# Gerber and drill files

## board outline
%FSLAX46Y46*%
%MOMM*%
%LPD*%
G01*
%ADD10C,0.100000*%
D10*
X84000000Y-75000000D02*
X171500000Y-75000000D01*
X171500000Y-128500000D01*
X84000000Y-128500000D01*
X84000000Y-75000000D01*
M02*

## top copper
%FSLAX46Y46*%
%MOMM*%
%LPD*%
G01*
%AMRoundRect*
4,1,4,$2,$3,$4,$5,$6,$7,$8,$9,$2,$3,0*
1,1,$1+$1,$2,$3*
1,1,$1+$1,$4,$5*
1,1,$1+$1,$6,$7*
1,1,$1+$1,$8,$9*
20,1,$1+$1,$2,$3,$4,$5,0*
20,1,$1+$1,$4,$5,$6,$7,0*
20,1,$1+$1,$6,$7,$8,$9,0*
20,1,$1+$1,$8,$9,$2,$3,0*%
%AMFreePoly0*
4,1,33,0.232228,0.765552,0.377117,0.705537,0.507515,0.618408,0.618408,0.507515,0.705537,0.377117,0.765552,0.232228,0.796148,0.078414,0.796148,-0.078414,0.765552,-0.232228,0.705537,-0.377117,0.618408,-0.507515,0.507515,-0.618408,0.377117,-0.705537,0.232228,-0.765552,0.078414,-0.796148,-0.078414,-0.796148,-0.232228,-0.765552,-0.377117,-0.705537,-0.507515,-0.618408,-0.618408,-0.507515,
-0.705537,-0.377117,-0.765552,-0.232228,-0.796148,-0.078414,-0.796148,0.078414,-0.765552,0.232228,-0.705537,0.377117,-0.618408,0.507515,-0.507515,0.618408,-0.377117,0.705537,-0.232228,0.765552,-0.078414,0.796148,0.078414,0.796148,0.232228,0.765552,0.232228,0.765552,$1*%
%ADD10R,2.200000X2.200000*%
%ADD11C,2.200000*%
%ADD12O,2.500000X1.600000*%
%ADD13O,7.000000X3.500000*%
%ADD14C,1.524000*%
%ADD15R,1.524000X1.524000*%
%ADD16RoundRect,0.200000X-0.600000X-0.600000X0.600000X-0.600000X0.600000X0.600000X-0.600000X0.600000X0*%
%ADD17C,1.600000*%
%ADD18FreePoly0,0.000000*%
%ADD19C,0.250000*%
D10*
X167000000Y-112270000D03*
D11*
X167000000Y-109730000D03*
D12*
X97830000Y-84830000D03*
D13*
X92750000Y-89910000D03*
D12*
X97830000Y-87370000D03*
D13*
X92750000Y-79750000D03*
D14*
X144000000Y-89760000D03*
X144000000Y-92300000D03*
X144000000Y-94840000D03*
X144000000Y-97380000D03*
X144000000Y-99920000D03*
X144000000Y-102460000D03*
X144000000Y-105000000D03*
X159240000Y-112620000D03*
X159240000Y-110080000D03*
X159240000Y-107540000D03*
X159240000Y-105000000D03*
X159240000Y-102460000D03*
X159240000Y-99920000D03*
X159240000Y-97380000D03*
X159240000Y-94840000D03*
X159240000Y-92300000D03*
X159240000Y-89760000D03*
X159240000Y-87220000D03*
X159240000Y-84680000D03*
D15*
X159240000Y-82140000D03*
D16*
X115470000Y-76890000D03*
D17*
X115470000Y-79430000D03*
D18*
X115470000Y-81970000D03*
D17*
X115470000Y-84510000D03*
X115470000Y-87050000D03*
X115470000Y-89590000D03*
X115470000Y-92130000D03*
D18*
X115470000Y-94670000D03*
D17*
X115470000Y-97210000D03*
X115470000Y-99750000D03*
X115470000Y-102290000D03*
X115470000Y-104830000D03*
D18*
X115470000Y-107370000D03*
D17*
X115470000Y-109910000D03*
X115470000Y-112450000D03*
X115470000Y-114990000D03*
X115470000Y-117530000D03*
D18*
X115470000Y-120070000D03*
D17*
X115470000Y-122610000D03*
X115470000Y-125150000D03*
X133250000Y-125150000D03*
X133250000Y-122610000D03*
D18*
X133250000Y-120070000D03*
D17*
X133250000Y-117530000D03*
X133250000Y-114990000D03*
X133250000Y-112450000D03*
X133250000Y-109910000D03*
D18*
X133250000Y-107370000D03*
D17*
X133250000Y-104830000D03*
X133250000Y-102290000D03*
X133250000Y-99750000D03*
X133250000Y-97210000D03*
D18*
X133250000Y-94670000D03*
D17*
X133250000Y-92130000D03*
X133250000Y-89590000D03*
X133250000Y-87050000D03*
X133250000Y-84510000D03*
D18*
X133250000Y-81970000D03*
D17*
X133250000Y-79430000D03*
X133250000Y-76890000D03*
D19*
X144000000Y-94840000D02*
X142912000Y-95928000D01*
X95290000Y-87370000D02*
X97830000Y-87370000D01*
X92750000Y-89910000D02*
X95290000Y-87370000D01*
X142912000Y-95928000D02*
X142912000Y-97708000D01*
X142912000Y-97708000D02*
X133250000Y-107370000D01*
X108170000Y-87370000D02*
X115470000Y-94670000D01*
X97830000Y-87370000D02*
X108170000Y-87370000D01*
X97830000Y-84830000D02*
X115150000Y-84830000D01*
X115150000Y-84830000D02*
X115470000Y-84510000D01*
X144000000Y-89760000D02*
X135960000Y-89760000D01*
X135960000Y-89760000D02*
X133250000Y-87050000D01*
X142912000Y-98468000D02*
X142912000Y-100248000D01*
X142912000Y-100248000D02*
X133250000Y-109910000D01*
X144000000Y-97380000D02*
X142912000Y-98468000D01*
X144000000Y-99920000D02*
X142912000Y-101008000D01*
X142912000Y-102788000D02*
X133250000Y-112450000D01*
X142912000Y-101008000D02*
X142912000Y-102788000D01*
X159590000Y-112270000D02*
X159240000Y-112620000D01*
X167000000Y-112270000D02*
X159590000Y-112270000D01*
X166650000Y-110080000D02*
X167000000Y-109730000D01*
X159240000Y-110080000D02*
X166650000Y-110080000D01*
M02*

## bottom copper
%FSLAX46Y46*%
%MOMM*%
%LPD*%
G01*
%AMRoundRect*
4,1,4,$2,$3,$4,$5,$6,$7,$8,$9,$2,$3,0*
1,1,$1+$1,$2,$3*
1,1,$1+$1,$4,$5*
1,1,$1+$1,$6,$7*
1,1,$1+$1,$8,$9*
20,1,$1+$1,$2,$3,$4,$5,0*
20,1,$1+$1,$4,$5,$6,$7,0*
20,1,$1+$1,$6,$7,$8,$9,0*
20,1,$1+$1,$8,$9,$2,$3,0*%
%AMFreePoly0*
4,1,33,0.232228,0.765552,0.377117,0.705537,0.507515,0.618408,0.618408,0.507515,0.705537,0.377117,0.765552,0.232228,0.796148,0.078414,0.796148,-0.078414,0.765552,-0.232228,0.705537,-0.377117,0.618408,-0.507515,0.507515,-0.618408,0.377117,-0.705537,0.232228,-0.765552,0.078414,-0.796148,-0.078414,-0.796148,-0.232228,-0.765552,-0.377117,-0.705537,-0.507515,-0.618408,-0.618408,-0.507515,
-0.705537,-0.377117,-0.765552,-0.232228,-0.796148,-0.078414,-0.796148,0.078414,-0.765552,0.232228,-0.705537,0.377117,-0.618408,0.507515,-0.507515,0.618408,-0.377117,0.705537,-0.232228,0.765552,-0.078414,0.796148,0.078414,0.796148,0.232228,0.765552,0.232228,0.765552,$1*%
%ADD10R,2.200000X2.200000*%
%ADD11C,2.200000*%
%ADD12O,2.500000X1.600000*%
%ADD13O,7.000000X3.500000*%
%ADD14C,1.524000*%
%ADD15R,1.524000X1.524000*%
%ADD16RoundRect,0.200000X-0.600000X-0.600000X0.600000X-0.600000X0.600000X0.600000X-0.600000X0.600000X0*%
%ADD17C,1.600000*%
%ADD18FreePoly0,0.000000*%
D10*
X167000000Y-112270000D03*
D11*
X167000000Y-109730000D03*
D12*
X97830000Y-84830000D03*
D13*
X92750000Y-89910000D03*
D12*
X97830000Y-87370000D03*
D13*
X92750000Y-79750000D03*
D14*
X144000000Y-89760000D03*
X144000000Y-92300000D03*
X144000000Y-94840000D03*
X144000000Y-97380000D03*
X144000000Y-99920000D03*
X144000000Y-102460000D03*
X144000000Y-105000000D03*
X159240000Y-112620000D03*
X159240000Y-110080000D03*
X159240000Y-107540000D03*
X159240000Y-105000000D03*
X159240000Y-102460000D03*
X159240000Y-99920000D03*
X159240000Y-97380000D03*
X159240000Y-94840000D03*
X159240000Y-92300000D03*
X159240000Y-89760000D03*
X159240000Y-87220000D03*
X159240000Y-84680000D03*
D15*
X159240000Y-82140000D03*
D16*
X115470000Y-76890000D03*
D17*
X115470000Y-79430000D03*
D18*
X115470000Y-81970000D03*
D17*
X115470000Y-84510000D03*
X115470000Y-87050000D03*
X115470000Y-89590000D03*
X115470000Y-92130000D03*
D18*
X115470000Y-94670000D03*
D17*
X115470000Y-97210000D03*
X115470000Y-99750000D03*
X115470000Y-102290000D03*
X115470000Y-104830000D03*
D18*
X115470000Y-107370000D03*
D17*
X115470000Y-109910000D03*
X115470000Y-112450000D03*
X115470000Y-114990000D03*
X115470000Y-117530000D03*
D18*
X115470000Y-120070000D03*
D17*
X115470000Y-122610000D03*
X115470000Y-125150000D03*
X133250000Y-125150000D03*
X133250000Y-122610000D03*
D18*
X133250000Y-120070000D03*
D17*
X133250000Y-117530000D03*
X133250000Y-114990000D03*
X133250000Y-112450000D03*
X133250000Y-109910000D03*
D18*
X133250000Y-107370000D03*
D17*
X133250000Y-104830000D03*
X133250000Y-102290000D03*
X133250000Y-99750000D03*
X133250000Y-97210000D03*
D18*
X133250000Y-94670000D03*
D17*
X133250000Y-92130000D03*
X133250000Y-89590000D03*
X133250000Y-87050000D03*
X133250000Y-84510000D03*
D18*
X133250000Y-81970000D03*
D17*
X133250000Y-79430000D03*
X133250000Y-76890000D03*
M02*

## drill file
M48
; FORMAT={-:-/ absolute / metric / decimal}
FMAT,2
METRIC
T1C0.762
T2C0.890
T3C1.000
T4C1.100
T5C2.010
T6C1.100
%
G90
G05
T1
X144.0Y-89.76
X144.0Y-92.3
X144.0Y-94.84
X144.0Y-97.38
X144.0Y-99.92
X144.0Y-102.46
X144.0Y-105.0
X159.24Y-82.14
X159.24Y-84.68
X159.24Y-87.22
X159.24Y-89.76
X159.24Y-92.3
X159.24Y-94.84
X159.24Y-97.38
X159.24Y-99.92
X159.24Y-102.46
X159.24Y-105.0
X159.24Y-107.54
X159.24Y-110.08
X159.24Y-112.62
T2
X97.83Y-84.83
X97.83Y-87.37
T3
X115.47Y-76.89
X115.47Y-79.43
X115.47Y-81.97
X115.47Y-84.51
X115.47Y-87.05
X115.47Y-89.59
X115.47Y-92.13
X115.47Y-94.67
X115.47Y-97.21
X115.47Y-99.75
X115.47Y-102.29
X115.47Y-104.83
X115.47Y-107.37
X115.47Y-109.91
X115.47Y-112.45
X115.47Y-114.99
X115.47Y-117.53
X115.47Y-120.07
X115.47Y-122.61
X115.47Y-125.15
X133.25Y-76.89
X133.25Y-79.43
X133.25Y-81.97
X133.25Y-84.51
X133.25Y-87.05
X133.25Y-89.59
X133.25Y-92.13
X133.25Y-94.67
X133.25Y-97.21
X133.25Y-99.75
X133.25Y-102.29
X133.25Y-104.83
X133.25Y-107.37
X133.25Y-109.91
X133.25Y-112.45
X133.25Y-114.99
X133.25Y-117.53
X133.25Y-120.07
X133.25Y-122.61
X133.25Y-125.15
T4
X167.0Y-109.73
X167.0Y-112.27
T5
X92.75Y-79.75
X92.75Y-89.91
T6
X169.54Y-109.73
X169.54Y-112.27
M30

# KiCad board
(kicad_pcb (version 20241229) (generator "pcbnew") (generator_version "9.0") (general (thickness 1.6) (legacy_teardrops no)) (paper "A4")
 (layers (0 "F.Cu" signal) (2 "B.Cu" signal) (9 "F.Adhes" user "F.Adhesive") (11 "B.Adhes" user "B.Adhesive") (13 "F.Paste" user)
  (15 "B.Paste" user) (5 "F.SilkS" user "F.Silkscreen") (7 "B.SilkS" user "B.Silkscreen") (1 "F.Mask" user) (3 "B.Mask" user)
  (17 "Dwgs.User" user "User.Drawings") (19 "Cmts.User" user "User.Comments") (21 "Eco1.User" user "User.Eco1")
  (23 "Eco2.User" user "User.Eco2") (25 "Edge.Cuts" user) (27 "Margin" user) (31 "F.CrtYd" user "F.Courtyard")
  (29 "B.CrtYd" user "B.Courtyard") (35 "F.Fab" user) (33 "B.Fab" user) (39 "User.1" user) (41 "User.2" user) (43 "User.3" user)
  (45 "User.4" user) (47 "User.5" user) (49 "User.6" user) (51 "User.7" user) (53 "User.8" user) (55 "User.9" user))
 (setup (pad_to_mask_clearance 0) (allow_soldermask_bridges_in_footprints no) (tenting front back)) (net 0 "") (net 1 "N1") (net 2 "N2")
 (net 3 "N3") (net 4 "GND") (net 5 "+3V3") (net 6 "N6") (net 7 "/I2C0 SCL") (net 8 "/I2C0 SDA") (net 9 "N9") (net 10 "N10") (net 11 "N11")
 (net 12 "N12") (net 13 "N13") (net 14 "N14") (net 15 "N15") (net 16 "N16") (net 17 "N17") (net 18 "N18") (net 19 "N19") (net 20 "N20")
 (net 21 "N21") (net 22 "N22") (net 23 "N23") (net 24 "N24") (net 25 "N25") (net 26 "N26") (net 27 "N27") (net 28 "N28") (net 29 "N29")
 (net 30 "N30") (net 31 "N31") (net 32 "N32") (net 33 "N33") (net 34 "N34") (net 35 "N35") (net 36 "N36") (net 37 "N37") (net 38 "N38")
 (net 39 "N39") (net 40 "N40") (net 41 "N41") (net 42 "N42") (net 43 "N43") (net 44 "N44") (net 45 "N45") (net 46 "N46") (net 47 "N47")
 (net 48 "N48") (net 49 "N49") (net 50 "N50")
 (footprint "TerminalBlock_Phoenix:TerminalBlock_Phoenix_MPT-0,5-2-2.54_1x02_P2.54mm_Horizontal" (layer "F.Cu") (at 167 112.27 90)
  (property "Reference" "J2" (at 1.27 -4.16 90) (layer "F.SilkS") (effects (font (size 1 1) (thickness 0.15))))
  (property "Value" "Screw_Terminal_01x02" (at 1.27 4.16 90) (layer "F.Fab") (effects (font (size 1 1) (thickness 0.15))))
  (pad "" np_thru_hole circle (at 0 2.54 90) (size 1.1 1.1) (drill 1.1) (layers "*.Cu" "*.Mask"))
  (pad "" np_thru_hole circle (at 2.54 2.54 90) (size 1.1 1.1) (drill 1.1) (layers "*.Cu" "*.Mask"))
  (pad "1" thru_hole rect (at 0 0 90) (size 2.2 2.2) (drill 1.1) (layers "*.Cu" "*.Mask") (remove_unused_layers no) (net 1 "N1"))
  (pad "2" thru_hole circle (at 2.54 0 90) (size 2.2 2.2) (drill 1.1) (layers "*.Cu" "*.Mask") (remove_unused_layers no) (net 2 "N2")))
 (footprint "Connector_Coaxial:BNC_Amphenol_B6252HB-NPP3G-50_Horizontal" (layer "F.Cu") (at 97.83 84.83 90)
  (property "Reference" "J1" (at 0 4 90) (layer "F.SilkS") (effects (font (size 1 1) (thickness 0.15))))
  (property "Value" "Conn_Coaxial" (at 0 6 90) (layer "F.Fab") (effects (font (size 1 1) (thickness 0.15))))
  (pad "1" thru_hole oval (at 0 0 90) (size 1.6 2.5) (drill 0.89) (layers "*.Cu" "*.Mask") (remove_unused_layers no) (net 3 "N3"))
  (pad "2" thru_hole oval (at -5.08 -5.08 90) (size 3.5 7) (drill 2.01) (layers "*.Cu" "*.Mask") (remove_unused_layers no) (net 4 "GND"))
  (pad "2" thru_hole oval (at -2.54 0 90) (size 1.6 2.5) (drill 0.89) (layers "*.Cu" "*.Mask") (remove_unused_layers no) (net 4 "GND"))
  (pad "2" thru_hole oval (at 5.08 -5.08 90) (size 3.5 7) (drill 2.01) (layers "*.Cu" "*.Mask") (remove_unused_layers no) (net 4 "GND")))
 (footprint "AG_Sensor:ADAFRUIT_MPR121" (layer "F.Cu") (at 152.89 94.84 -90)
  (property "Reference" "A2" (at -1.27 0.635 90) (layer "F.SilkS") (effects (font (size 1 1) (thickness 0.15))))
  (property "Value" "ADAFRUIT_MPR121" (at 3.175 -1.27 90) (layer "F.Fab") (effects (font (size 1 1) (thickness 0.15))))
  (pad "1" thru_hole circle (at -5.08 8.89 270) (size 1.524 1.524) (drill 0.762) (layers "*.Cu" "*.Mask") (remove_unused_layers no)
   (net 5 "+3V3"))
  (pad "2" thru_hole circle (at -2.54 8.89 270) (size 1.524 1.524) (drill 0.762) (layers "*.Cu" "*.Mask") (remove_unused_layers no)
   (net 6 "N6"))
  (pad "3" thru_hole circle (at 0 8.89 270) (size 1.524 1.524) (drill 0.762) (layers "*.Cu" "*.Mask") (remove_unused_layers no)
   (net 4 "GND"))
  (pad "4" thru_hole circle (at 2.54 8.89 270) (size 1.524 1.524) (drill 0.762) (layers "*.Cu" "*.Mask") (remove_unused_layers no)
   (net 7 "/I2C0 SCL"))
  (pad "5" thru_hole circle (at 5.08 8.89 270) (size 1.524 1.524) (drill 0.762) (layers "*.Cu" "*.Mask") (remove_unused_layers no)
   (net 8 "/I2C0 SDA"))
  (pad "6" thru_hole circle (at 7.62 8.89 270) (size 1.524 1.524) (drill 0.762) (layers "*.Cu" "*.Mask") (remove_unused_layers no)
   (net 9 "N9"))
  (pad "7" thru_hole circle (at 10.16 8.89 270) (size 1.524 1.524) (drill 0.762) (layers "*.Cu" "*.Mask") (remove_unused_layers no)
   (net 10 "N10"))
  (pad "8" thru_hole circle (at 17.78 -6.35 270) (size 1.524 1.524) (drill 0.762) (layers "*.Cu" "*.Mask") (remove_unused_layers no)
   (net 1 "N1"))
  (pad "9" thru_hole circle (at 15.24 -6.35 270) (size 1.524 1.524) (drill 0.762) (layers "*.Cu" "*.Mask") (remove_unused_layers no)
   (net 2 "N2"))
  (pad "10" thru_hole circle (at 12.7 -6.35 270) (size 1.524 1.524) (drill 0.762) (layers "*.Cu" "*.Mask") (remove_unused_layers no)
   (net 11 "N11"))
  (pad "11" thru_hole circle (at 10.16 -6.35) (size 1.524 1.524) (drill 0.762) (layers "*.Cu" "*.Mask") (remove_unused_layers no)
   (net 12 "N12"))
  (pad "12" thru_hole circle (at 7.62 -6.35 270) (size 1.524 1.524) (drill 0.762) (layers "*.Cu" "*.Mask") (remove_unused_layers no)
   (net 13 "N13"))
  (pad "13" thru_hole circle (at 5.08 -6.35 270) (size 1.524 1.524) (drill 0.762) (layers "*.Cu" "*.Mask") (remove_unused_layers no)
   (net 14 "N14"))
  (pad "14" thru_hole circle (at 2.54 -6.35 270) (size 1.524 1.524) (drill 0.762) (layers "*.Cu" "*.Mask") (remove_unused_layers no)
   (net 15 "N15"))
  (pad "15" thru_hole circle (at 0 -6.35 270) (size 1.524 1.524) (drill 0.762) (layers "*.Cu" "*.Mask") (remove_unused_layers no)
   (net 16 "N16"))
  (pad "16" thru_hole circle (at -2.54 -6.35 270) (size 1.524 1.524) (drill 0.762) (layers "*.Cu" "*.Mask") (remove_unused_layers no)
   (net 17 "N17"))
  (pad "17" thru_hole circle (at -5.08 -6.35 270) (size 1.524 1.524) (drill 0.762) (layers "*.Cu" "*.Mask") (remove_unused_layers no)
   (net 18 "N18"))
  (pad "18" thru_hole circle (at -7.62 -6.35 270) (size 1.524 1.524) (drill 0.762) (layers "*.Cu" "*.Mask") (remove_unused_layers no)
   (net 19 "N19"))
  (pad "19" thru_hole circle (at -10.16 -6.35 270) (size 1.524 1.524) (drill 0.762) (layers "*.Cu" "*.Mask") (remove_unused_layers no)
   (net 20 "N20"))
  (pad "20" thru_hole rect (at -12.7 -6.35 270) (size 1.524 1.524) (drill 0.762) (layers "*.Cu" "*.Mask") (remove_unused_layers no)
   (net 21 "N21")))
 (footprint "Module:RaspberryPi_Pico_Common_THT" (layer "F.Cu") (at 115.47 76.89)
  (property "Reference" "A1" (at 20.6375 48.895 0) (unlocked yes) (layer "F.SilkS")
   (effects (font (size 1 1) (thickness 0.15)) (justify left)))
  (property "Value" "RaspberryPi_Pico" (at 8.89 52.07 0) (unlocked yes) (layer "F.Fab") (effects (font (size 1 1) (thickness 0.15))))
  (pad "1" thru_hole roundrect (at 0 0) (size 1.6 1.6) (drill 1) (layers "*.Cu" "*.Mask") (remove_unused_layers no) (roundrect_rratio 0.125)
   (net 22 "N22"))
  (pad "2" thru_hole circle (at 0 2.54) (size 1.6 1.6) (drill 1) (layers "*.Cu" "*.Mask") (remove_unused_layers no) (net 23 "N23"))
  (pad "3" thru_hole custom (at 0 5.08) (size 1.6 1.6) (drill 1) (layers "*.Cu" "*.Mask") (remove_unused_layers no) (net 4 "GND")
   (options (clearance outline) (anchor circle)) (primitives))
  (pad "4" thru_hole circle (at 0 7.62) (size 1.6 1.6) (drill 1) (layers "*.Cu" "*.Mask") (remove_unused_layers no) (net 3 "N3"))
  (pad "5" thru_hole circle (at 0 10.16) (size 1.6 1.6) (drill 1) (layers "*.Cu" "*.Mask") (remove_unused_layers no) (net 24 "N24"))
  (pad "6" thru_hole circle (at 0 12.7) (size 1.6 1.6) (drill 1) (layers "*.Cu" "*.Mask") (remove_unused_layers no) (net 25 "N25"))
  (pad "7" thru_hole circle (at 0 15.24) (size 1.6 1.6) (drill 1) (layers "*.Cu" "*.Mask") (remove_unused_layers no) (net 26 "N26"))
  (pad "8" thru_hole custom (at 0 17.78) (size 1.6 1.6) (drill 1) (layers "*.Cu" "*.Mask") (remove_unused_layers no) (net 4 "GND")
   (options (clearance outline) (anchor circle)) (primitives))
  (pad "9" thru_hole circle (at 0 20.32) (size 1.6 1.6) (drill 1) (layers "*.Cu" "*.Mask") (remove_unused_layers no) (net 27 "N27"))
  (pad "10" thru_hole circle (at 0 22.86) (size 1.6 1.6) (drill 1) (layers "*.Cu" "*.Mask") (remove_unused_layers no) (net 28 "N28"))
  (pad "11" thru_hole circle (at 0 25.4) (size 1.6 1.6) (drill 1) (layers "*.Cu" "*.Mask") (remove_unused_layers no) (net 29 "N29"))
  (pad "12" thru_hole circle (at 0 27.94) (size 1.6 1.6) (drill 1) (layers "*.Cu" "*.Mask") (remove_unused_layers no) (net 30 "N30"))
  (pad "13" thru_hole custom (at 0 30.48) (size 1.6 1.6) (drill 1) (layers "*.Cu" "*.Mask") (remove_unused_layers no) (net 4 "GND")
   (options (clearance outline) (anchor circle)) (primitives))
  (pad "14" thru_hole circle (at 0 33.02) (size 1.6 1.6) (drill 1) (layers "*.Cu" "*.Mask") (remove_unused_layers no) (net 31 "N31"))
  (pad "15" thru_hole circle (at 0 35.56) (size 1.6 1.6) (drill 1) (layers "*.Cu" "*.Mask") (remove_unused_layers no) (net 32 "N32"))
  (pad "16" thru_hole circle (at 0 38.1) (size 1.6 1.6) (drill 1) (layers "*.Cu" "*.Mask") (remove_unused_layers no) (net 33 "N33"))
  (pad "17" thru_hole circle (at 0 40.64) (size 1.6 1.6) (drill 1) (layers "*.Cu" "*.Mask") (remove_unused_layers no) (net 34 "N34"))
  (pad "18" thru_hole custom (at 0 43.18) (size 1.6 1.6) (drill 1) (layers "*.Cu" "*.Mask") (remove_unused_layers no) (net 4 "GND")
   (options (clearance outline) (anchor circle)) (primitives))
  (pad "19" thru_hole circle (at 0 45.72) (size 1.6 1.6) (drill 1) (layers "*.Cu" "*.Mask") (remove_unused_layers no) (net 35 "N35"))
  (pad "20" thru_hole circle (at 0 48.26) (size 1.6 1.6) (drill 1) (layers "*.Cu" "*.Mask") (remove_unused_layers no) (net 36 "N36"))
  (pad "21" thru_hole circle (at 17.78 48.26) (size 1.6 1.6) (drill 1) (layers "*.Cu" "*.Mask") (remove_unused_layers no) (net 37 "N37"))
  (pad "22" thru_hole circle (at 17.78 45.72) (size 1.6 1.6) (drill 1) (layers "*.Cu" "*.Mask") (remove_unused_layers no) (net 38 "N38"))
  (pad "23" thru_hole custom (at 17.78 43.18) (size 1.6 1.6) (drill 1) (layers "*.Cu" "*.Mask") (remove_unused_layers no) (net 4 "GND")
   (options (clearance outline) (anchor circle)) (primitives))
  (pad "24" thru_hole circle (at 17.78 40.64) (size 1.6 1.6) (drill 1) (layers "*.Cu" "*.Mask") (remove_unused_layers no) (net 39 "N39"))
  (pad "25" thru_hole circle (at 17.78 38.1) (size 1.6 1.6) (drill 1) (layers "*.Cu" "*.Mask") (remove_unused_layers no) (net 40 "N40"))
  (pad "26" thru_hole circle (at 17.78 35.56) (size 1.6 1.6) (drill 1) (layers "*.Cu" "*.Mask") (remove_unused_layers no)
   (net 8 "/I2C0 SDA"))
  (pad "27" thru_hole circle (at 17.78 33.02) (size 1.6 1.6) (drill 1) (layers "*.Cu" "*.Mask") (remove_unused_layers no)
   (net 7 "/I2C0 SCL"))
  (pad "28" thru_hole custom (at 17.78 30.48) (size 1.6 1.6) (drill 1) (layers "*.Cu" "*.Mask") (remove_unused_layers no) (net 4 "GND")
   (options (clearance outline) (anchor circle)) (primitives))
  (pad "29" thru_hole circle (at 17.78 27.94) (size 1.6 1.6) (drill 1) (layers "*.Cu" "*.Mask") (remove_unused_layers no) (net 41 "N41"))
  (pad "30" thru_hole circle (at 17.78 25.4) (size 1.6 1.6) (drill 1) (layers "*.Cu" "*.Mask") (remove_unused_layers no) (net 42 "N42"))
  (pad "31" thru_hole circle (at 17.78 22.86) (size 1.6 1.6) (drill 1) (layers "*.Cu" "*.Mask") (remove_unused_layers no) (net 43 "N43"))
  (pad "32" thru_hole circle (at 17.78 20.32) (size 1.6 1.6) (drill 1) (layers "*.Cu" "*.Mask") (remove_unused_layers no) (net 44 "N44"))
  (pad "33" thru_hole custom (at 17.78 17.78) (size 1.6 1.6) (drill 1) (layers "*.Cu" "*.Mask") (remove_unused_layers no) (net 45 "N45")
   (options (clearance outline) (anchor circle)) (primitives))
  (pad "34" thru_hole circle (at 17.78 15.24) (size 1.6 1.6) (drill 1) (layers "*.Cu" "*.Mask") (remove_unused_layers no) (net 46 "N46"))
  (pad "35" thru_hole circle (at 17.78 12.7) (size 1.6 1.6) (drill 1) (layers "*.Cu" "*.Mask") (remove_unused_layers no) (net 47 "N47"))
  (pad "36" thru_hole circle (at 17.78 10.16) (size 1.6 1.6) (drill 1) (layers "*.Cu" "*.Mask") (remove_unused_layers no) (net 5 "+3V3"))
  (pad "37" thru_hole circle (at 17.78 7.62) (size 1.6 1.6) (drill 1) (layers "*.Cu" "*.Mask") (remove_unused_layers no) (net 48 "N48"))
  (pad "38" thru_hole custom (at 17.78 5.08) (size 1.6 1.6) (drill 1) (layers "*.Cu" "*.Mask") (remove_unused_layers no) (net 4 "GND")
   (options (clearance outline) (anchor circle)) (primitives))
  (pad "39" thru_hole circle (at 17.78 2.54) (size 1.6 1.6) (drill 1) (layers "*.Cu" "*.Mask") (remove_unused_layers no) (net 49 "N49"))
  (pad "40" thru_hole circle (at 17.78 0) (size 1.6 1.6) (drill 1) (layers "*.Cu" "*.Mask") (remove_unused_layers no) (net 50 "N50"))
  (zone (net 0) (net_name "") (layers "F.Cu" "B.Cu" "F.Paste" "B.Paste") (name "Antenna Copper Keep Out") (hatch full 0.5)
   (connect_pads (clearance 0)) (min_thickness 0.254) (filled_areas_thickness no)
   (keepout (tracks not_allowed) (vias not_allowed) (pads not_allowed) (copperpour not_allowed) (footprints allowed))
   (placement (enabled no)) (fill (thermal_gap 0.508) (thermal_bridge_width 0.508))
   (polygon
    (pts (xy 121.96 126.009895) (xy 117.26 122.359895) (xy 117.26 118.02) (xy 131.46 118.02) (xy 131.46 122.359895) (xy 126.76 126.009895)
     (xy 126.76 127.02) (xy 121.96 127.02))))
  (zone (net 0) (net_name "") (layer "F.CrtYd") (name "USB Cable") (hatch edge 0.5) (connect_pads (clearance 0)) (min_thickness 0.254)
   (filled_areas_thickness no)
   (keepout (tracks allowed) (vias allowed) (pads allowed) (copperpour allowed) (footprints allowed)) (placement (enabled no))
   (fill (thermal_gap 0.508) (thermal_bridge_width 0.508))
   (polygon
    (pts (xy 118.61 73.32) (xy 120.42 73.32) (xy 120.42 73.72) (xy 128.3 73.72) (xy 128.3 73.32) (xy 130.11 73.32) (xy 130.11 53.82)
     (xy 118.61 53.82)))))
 (gr_rect (start 84 75) (end 171.5 128.5) (stroke (width 0.1) (type default)) (fill no) (layer "Edge.Cuts"))
 (segment (start 144 94.84) (end 142.912 95.928) (width 0.25) (layer "F.Cu") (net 4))
 (segment (start 95.29 87.37) (end 97.83 87.37) (width 0.25) (layer "F.Cu") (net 4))
 (segment (start 92.75 89.91) (end 95.29 87.37) (width 0.25) (layer "F.Cu") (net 4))
 (segment (start 142.912 95.928) (end 142.912 97.708) (width 0.25) (layer "F.Cu") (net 4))
 (segment (start 142.912 97.708) (end 133.25 107.37) (width 0.25) (layer "F.Cu") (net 4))
 (segment (start 108.17 87.37) (end 115.47 94.67) (width 0.25) (layer "F.Cu") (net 4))
 (segment (start 97.83 87.37) (end 108.17 87.37) (width 0.25) (layer "F.Cu") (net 4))
 (segment (start 97.83 84.83) (end 115.15 84.83) (width 0.25) (layer "F.Cu") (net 3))
 (segment (start 115.15 84.83) (end 115.47 84.51) (width 0.25) (layer "F.Cu") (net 3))
 (segment (start 144 89.76) (end 135.96 89.76) (width 0.25) (layer "F.Cu") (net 5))
 (segment (start 135.96 89.76) (end 133.25 87.05) (width 0.25) (layer "F.Cu") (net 5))
 (segment (start 142.912 98.468) (end 142.912 100.248) (width 0.25) (layer "F.Cu") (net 7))
 (segment (start 142.912 100.248) (end 133.25 109.91) (width 0.25) (layer "F.Cu") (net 7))
 (segment (start 144 97.38) (end 142.912 98.468) (width 0.25) (layer "F.Cu") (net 7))
 (segment (start 144 99.92) (end 142.912 101.008) (width 0.25) (layer "F.Cu") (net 8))
 (segment (start 142.912 102.788) (end 133.25 112.45) (width 0.25) (layer "F.Cu") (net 8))
 (segment (start 142.912 101.008) (end 142.912 102.788) (width 0.25) (layer "F.Cu") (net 8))
 (segment (start 159.59 112.27) (end 159.24 112.62) (width 0.25) (layer "F.Cu") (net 1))
 (segment (start 167 112.27) (end 159.59 112.27) (width 0.25) (layer "F.Cu") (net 1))
 (segment (start 166.65 110.08) (end 167 109.73) (width 0.25) (layer "F.Cu") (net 2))
 (segment (start 159.24 110.08) (end 166.65 110.08) (width 0.25) (layer "F.Cu") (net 2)))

